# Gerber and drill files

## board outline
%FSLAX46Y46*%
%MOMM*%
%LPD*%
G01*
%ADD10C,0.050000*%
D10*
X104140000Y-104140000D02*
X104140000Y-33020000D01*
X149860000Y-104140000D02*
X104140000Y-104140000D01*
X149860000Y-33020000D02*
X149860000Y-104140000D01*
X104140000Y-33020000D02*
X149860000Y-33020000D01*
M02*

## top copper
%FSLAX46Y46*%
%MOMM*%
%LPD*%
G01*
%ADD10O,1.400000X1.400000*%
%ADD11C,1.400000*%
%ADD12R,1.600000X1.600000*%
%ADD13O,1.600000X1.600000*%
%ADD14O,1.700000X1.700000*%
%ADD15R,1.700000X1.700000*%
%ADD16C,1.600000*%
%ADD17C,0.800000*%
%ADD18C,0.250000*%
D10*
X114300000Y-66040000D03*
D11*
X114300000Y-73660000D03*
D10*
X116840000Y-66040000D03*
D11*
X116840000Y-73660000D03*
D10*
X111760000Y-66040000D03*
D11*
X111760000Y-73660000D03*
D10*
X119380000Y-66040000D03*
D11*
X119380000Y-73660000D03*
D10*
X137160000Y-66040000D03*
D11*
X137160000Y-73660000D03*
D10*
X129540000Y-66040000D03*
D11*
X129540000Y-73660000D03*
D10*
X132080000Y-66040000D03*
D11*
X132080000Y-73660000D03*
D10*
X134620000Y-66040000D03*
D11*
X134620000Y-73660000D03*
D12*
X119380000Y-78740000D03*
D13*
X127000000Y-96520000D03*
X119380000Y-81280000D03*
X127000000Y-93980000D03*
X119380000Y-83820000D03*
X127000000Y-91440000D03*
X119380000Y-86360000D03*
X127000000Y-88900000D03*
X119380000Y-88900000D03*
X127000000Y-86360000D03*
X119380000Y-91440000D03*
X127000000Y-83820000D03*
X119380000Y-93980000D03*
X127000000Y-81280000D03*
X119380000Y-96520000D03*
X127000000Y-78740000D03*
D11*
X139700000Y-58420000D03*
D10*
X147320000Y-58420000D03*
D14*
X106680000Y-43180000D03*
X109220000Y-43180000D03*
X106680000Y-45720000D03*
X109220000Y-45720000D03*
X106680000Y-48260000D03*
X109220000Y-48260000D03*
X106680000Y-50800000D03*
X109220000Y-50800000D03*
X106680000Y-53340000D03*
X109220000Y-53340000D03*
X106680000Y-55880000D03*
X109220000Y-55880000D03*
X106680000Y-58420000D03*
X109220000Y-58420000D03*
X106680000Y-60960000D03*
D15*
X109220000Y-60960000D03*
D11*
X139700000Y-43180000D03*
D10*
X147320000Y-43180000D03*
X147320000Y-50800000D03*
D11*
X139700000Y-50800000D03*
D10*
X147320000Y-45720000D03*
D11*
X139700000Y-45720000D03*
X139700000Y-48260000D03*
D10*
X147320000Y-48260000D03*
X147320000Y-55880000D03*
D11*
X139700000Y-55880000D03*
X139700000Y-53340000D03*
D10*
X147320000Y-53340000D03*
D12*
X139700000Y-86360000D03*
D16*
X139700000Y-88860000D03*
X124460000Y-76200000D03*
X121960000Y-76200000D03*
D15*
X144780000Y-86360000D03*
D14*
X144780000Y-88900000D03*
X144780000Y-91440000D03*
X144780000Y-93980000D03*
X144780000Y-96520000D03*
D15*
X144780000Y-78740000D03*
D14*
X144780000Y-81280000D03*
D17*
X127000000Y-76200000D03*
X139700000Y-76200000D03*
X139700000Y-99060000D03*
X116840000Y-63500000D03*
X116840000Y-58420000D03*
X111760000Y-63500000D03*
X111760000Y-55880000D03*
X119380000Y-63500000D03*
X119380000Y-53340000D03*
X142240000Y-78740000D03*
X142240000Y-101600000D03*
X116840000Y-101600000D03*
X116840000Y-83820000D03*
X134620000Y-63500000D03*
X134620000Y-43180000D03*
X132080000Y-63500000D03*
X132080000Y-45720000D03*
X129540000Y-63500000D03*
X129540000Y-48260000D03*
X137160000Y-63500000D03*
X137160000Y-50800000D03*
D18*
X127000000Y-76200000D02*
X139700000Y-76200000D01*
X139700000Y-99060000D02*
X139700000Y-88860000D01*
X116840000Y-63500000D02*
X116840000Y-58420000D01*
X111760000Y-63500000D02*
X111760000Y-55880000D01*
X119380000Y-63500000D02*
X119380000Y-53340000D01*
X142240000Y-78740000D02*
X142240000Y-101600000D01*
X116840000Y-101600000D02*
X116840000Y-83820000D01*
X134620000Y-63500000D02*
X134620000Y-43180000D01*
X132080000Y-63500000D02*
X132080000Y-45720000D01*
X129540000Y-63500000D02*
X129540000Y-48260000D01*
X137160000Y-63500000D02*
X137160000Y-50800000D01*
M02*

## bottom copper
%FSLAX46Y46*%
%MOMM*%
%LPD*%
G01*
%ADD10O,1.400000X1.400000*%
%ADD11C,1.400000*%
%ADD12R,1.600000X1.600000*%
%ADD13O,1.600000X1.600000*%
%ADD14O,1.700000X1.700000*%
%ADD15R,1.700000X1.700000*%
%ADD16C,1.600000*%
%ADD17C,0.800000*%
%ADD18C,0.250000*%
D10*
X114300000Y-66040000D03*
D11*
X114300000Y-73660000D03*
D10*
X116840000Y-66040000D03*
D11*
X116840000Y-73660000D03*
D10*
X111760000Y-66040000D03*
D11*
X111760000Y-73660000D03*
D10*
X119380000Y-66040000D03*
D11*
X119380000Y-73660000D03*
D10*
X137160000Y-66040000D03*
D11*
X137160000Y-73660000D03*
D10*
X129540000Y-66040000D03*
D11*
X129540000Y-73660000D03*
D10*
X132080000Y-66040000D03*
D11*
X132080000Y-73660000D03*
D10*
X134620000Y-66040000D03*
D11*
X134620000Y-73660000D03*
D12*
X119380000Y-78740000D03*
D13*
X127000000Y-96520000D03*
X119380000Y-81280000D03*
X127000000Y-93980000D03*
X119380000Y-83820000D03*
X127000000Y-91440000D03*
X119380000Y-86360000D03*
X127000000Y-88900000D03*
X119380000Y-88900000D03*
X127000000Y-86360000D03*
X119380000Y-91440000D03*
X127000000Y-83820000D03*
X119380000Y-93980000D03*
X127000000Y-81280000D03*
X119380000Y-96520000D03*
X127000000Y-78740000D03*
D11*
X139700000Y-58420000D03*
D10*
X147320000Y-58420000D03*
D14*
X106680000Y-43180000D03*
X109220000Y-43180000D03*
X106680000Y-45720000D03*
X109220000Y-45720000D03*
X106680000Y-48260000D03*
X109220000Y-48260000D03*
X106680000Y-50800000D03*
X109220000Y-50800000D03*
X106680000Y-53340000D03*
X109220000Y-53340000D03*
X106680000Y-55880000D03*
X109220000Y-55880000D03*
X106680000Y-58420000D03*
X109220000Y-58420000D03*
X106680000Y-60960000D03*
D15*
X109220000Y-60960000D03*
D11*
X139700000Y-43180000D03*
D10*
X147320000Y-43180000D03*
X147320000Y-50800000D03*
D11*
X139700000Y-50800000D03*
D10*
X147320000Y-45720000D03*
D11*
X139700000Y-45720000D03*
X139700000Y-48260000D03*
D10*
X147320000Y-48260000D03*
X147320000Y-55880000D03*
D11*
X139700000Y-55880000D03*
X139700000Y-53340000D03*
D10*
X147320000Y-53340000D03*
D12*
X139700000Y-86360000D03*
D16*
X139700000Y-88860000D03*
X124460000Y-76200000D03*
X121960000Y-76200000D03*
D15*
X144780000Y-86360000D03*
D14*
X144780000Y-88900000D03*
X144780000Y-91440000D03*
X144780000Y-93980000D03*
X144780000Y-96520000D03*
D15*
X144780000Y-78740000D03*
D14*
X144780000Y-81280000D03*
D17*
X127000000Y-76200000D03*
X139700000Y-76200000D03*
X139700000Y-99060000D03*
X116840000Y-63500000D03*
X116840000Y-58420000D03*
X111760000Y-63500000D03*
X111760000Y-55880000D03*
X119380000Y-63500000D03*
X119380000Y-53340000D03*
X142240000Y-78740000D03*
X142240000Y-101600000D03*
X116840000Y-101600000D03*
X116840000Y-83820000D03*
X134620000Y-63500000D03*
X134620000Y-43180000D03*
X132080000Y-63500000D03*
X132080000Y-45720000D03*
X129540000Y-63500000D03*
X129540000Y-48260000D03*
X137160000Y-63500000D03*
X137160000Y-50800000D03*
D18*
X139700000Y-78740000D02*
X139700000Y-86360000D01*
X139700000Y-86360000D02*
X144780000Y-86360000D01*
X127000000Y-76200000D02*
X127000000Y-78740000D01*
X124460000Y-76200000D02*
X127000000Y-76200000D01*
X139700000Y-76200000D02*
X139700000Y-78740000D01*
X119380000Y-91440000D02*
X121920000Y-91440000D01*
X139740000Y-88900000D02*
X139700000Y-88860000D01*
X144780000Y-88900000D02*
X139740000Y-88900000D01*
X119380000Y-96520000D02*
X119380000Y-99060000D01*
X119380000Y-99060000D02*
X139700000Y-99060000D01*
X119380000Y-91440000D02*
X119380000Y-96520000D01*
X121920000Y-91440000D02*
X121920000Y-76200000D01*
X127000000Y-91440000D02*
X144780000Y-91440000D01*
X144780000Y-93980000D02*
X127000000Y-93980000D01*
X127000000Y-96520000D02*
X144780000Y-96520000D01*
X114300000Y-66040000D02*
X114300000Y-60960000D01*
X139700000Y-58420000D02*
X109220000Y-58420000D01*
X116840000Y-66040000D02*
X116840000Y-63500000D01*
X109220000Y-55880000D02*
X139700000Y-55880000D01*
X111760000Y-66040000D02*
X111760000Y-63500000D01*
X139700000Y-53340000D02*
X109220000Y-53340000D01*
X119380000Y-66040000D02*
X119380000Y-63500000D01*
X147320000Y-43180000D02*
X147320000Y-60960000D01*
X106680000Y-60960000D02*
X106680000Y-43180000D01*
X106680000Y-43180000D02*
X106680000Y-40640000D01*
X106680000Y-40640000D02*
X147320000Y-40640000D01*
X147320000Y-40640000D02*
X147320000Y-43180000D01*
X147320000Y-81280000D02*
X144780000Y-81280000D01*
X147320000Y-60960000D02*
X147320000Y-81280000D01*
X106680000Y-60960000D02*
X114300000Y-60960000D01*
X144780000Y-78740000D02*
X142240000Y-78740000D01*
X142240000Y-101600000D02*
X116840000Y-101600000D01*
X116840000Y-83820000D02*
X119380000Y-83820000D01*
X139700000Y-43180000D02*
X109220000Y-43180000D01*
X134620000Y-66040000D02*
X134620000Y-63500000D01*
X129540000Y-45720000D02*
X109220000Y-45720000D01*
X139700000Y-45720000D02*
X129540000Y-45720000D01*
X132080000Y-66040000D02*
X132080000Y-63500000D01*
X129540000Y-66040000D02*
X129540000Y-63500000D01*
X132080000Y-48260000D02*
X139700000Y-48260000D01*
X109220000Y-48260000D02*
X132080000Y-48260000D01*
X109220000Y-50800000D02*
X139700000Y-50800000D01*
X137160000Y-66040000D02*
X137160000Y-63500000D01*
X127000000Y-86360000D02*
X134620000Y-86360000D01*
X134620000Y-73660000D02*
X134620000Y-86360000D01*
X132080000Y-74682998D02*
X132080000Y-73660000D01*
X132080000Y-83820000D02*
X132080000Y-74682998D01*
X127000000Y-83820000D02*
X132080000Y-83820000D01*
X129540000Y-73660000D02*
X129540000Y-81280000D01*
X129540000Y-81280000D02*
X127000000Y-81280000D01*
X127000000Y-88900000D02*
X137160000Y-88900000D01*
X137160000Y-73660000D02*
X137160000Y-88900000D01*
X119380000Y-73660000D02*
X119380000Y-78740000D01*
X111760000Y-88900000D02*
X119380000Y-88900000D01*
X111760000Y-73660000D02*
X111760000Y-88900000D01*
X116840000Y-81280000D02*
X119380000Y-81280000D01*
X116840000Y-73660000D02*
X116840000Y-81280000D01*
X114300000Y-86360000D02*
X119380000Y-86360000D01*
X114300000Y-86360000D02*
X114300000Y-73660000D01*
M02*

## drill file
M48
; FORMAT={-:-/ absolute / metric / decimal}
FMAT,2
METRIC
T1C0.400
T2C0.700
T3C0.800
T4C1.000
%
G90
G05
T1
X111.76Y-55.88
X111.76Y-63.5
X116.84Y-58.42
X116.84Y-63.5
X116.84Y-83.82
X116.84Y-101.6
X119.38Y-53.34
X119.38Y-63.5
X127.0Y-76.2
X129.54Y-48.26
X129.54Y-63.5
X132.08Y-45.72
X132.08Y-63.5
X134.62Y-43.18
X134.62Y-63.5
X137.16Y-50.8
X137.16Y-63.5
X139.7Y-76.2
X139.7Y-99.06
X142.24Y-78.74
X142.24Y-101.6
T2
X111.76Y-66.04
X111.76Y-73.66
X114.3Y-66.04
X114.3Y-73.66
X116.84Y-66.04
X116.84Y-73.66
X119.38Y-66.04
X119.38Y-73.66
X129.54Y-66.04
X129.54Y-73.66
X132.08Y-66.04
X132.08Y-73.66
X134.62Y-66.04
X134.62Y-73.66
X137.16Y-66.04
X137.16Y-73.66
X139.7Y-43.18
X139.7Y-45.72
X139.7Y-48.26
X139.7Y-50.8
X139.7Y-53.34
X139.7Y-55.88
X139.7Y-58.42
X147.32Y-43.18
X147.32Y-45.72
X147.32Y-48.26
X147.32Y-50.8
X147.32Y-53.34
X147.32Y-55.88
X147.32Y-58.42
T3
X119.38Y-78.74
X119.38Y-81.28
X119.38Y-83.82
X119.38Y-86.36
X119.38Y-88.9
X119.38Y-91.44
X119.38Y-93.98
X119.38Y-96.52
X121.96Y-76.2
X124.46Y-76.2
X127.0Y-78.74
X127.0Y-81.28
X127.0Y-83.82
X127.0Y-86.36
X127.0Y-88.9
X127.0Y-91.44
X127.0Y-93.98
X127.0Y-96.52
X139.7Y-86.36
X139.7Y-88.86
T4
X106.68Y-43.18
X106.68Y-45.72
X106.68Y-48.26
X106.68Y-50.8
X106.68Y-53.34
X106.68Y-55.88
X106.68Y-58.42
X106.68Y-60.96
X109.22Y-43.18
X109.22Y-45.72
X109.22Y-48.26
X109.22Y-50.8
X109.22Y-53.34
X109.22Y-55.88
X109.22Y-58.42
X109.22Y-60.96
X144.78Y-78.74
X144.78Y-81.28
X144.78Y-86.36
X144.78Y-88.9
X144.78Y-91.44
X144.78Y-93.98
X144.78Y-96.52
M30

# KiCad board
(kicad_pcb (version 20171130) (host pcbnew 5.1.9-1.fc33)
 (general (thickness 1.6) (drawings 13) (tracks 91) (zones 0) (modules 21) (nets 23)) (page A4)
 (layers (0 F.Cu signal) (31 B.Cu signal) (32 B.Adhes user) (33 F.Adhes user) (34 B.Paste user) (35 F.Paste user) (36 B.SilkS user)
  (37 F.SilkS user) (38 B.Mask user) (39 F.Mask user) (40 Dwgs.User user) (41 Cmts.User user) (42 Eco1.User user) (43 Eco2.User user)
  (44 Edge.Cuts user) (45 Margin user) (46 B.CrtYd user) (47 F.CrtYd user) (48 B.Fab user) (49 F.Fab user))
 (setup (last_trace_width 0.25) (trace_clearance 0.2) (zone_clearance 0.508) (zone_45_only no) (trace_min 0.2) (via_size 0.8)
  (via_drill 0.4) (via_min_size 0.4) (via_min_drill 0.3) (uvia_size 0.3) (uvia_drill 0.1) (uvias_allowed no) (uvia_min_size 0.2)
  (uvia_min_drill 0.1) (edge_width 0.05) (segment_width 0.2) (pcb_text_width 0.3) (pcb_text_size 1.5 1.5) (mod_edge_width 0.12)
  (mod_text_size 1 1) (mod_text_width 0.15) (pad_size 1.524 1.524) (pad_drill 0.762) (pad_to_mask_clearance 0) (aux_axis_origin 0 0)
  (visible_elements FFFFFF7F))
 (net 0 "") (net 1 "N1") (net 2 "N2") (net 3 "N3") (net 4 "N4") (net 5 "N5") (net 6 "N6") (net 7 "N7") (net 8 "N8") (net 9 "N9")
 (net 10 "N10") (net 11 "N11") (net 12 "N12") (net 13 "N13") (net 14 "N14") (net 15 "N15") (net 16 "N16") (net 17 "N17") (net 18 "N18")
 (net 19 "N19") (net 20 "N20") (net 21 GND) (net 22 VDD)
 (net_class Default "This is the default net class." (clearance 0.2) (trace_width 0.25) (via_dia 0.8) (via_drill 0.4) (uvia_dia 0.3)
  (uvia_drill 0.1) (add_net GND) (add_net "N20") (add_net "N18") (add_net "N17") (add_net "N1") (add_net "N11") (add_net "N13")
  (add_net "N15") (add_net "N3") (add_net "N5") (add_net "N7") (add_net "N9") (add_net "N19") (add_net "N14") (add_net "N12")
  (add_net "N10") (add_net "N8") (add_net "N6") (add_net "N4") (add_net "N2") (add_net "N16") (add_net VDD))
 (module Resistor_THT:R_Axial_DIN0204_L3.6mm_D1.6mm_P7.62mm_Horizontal (layer F.Cu) (at 114.3 73.66 90)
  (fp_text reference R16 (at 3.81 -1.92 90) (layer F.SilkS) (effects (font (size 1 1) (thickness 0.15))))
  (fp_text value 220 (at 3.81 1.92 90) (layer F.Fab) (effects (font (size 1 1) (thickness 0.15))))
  (pad 2 thru_hole oval (at 7.62 0 90) (size 1.4 1.4) (drill 0.7) (layers *.Cu *.Mask) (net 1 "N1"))
  (pad 1 thru_hole circle (at 0 0 90) (size 1.4 1.4) (drill 0.7) (layers *.Cu *.Mask) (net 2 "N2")))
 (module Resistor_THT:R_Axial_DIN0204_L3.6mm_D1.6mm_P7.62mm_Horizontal (layer F.Cu) (at 116.84 73.66 90)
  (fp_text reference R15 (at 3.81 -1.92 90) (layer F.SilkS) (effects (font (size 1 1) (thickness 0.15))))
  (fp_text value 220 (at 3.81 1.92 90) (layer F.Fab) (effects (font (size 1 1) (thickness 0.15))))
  (pad 2 thru_hole oval (at 7.62 0 90) (size 1.4 1.4) (drill 0.7) (layers *.Cu *.Mask) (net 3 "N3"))
  (pad 1 thru_hole circle (at 0 0 90) (size 1.4 1.4) (drill 0.7) (layers *.Cu *.Mask) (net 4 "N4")))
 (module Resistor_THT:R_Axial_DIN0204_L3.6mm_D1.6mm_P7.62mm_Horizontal (layer F.Cu) (at 111.76 73.66 90)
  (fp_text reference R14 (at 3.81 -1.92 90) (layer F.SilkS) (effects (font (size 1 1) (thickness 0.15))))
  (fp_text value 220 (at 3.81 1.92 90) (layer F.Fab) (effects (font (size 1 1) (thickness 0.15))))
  (pad 2 thru_hole oval (at 7.62 0 90) (size 1.4 1.4) (drill 0.7) (layers *.Cu *.Mask) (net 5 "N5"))
  (pad 1 thru_hole circle (at 0 0 90) (size 1.4 1.4) (drill 0.7) (layers *.Cu *.Mask) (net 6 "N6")))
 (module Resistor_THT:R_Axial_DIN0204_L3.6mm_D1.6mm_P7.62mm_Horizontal (layer F.Cu) (at 119.38 73.66 90)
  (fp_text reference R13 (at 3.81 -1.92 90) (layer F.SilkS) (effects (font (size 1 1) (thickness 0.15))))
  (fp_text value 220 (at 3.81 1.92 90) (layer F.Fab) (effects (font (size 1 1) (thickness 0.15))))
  (pad 2 thru_hole oval (at 7.62 0 90) (size 1.4 1.4) (drill 0.7) (layers *.Cu *.Mask) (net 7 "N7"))
  (pad 1 thru_hole circle (at 0 0 90) (size 1.4 1.4) (drill 0.7) (layers *.Cu *.Mask) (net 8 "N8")))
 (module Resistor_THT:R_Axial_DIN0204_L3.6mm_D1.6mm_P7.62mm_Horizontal (layer F.Cu) (at 137.16 73.66 90)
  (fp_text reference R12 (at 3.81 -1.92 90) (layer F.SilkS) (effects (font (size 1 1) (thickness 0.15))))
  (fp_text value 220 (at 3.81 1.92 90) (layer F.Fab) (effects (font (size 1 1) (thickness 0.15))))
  (pad 2 thru_hole oval (at 7.62 0 90) (size 1.4 1.4) (drill 0.7) (layers *.Cu *.Mask) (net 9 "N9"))
  (pad 1 thru_hole circle (at 0 0 90) (size 1.4 1.4) (drill 0.7) (layers *.Cu *.Mask) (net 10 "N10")))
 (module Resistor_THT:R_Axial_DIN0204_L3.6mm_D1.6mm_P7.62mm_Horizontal (layer F.Cu) (at 129.54 73.66 90)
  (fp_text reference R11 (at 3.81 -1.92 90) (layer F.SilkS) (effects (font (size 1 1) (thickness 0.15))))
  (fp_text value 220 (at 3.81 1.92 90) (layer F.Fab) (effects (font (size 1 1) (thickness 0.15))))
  (pad 2 thru_hole oval (at 7.62 0 90) (size 1.4 1.4) (drill 0.7) (layers *.Cu *.Mask) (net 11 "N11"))
  (pad 1 thru_hole circle (at 0 0 90) (size 1.4 1.4) (drill 0.7) (layers *.Cu *.Mask) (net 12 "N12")))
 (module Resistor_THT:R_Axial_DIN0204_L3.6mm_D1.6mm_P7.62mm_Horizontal (layer F.Cu) (at 132.08 73.66 90)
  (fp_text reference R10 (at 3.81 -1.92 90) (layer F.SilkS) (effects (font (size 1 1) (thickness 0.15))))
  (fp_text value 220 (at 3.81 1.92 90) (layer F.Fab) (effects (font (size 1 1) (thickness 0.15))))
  (pad 2 thru_hole oval (at 7.62 0 90) (size 1.4 1.4) (drill 0.7) (layers *.Cu *.Mask) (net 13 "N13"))
  (pad 1 thru_hole circle (at 0 0 90) (size 1.4 1.4) (drill 0.7) (layers *.Cu *.Mask) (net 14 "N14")))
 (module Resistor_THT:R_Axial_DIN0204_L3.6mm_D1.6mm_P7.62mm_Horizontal (layer F.Cu) (at 134.62 73.66 90)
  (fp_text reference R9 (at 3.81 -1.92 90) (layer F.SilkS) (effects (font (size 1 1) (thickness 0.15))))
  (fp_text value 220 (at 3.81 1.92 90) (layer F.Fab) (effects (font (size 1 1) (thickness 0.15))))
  (pad 2 thru_hole oval (at 7.62 0 90) (size 1.4 1.4) (drill 0.7) (layers *.Cu *.Mask) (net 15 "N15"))
  (pad 1 thru_hole circle (at 0 0 90) (size 1.4 1.4) (drill 0.7) (layers *.Cu *.Mask) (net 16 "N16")))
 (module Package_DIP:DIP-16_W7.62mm (layer F.Cu) (at 119.38 78.74)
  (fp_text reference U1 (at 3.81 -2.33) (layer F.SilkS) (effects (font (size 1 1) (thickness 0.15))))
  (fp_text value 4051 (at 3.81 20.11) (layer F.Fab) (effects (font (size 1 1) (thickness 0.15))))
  (pad 1 thru_hole rect (at 0 0) (size 1.6 1.6) (drill 0.8) (layers *.Cu *.Mask) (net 8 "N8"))
  (pad 9 thru_hole oval (at 7.62 17.78) (size 1.6 1.6) (drill 0.8) (layers *.Cu *.Mask) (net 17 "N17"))
  (pad 2 thru_hole oval (at 0 2.54) (size 1.6 1.6) (drill 0.8) (layers *.Cu *.Mask) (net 4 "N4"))
  (pad 10 thru_hole oval (at 7.62 15.24) (size 1.6 1.6) (drill 0.8) (layers *.Cu *.Mask) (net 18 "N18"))
  (pad 3 thru_hole oval (at 0 5.08) (size 1.6 1.6) (drill 0.8) (layers *.Cu *.Mask) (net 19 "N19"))
  (pad 11 thru_hole oval (at 7.62 12.7) (size 1.6 1.6) (drill 0.8) (layers *.Cu *.Mask) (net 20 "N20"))
  (pad 4 thru_hole oval (at 0 7.62) (size 1.6 1.6) (drill 0.8) (layers *.Cu *.Mask) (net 2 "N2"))
  (pad 12 thru_hole oval (at 7.62 10.16) (size 1.6 1.6) (drill 0.8) (layers *.Cu *.Mask) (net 10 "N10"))
  (pad 5 thru_hole oval (at 0 10.16) (size 1.6 1.6) (drill 0.8) (layers *.Cu *.Mask) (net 6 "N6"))
  (pad 13 thru_hole oval (at 7.62 7.62) (size 1.6 1.6) (drill 0.8) (layers *.Cu *.Mask) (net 16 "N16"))
  (pad 6 thru_hole oval (at 0 12.7) (size 1.6 1.6) (drill 0.8) (layers *.Cu *.Mask) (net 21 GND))
  (pad 14 thru_hole oval (at 7.62 5.08) (size 1.6 1.6) (drill 0.8) (layers *.Cu *.Mask) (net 14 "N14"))
  (pad 7 thru_hole oval (at 0 15.24) (size 1.6 1.6) (drill 0.8) (layers *.Cu *.Mask) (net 21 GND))
  (pad 15 thru_hole oval (at 7.62 2.54) (size 1.6 1.6) (drill 0.8) (layers *.Cu *.Mask) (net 12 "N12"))
  (pad 8 thru_hole oval (at 0 17.78) (size 1.6 1.6) (drill 0.8) (layers *.Cu *.Mask) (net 21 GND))
  (pad 16 thru_hole oval (at 7.62 0) (size 1.6 1.6) (drill 0.8) (layers *.Cu *.Mask) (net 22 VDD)))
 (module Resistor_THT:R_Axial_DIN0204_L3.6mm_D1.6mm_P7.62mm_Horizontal (layer F.Cu) (at 139.7 58.42)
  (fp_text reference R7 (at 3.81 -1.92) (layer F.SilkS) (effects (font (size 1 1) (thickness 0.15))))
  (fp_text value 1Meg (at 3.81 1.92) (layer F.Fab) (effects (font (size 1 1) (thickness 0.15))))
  (pad 1 thru_hole circle (at 0 0) (size 1.4 1.4) (drill 0.7) (layers *.Cu *.Mask) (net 3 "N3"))
  (pad 2 thru_hole oval (at 7.62 0) (size 1.4 1.4) (drill 0.7) (layers *.Cu *.Mask) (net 1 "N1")))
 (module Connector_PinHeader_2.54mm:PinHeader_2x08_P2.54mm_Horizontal (layer F.Cu) (at 109.22 60.96 180)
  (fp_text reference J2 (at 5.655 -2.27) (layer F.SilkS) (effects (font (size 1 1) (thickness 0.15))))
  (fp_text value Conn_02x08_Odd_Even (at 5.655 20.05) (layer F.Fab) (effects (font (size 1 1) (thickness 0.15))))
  (pad 16 thru_hole oval (at 2.54 17.78 180) (size 1.7 1.7) (drill 1) (layers *.Cu *.Mask) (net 1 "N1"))
  (pad 15 thru_hole oval (at 0 17.78 180) (size 1.7 1.7) (drill 1) (layers *.Cu *.Mask) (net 15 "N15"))
  (pad 14 thru_hole oval (at 2.54 15.24 180) (size 1.7 1.7) (drill 1) (layers *.Cu *.Mask) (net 1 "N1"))
  (pad 13 thru_hole oval (at 0 15.24 180) (size 1.7 1.7) (drill 1) (layers *.Cu *.Mask) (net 13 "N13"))
  (pad 12 thru_hole oval (at 2.54 12.7 180) (size 1.7 1.7) (drill 1) (layers *.Cu *.Mask) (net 1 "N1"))
  (pad 11 thru_hole oval (at 0 12.7 180) (size 1.7 1.7) (drill 1) (layers *.Cu *.Mask) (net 11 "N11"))
  (pad 10 thru_hole oval (at 2.54 10.16 180) (size 1.7 1.7) (drill 1) (layers *.Cu *.Mask) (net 1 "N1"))
  (pad 9 thru_hole oval (at 0 10.16 180) (size 1.7 1.7) (drill 1) (layers *.Cu *.Mask) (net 9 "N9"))
  (pad 8 thru_hole oval (at 2.54 7.62 180) (size 1.7 1.7) (drill 1) (layers *.Cu *.Mask) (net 1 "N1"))
  (pad 7 thru_hole oval (at 0 7.62 180) (size 1.7 1.7) (drill 1) (layers *.Cu *.Mask) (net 7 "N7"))
  (pad 6 thru_hole oval (at 2.54 5.08 180) (size 1.7 1.7) (drill 1) (layers *.Cu *.Mask) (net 1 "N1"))
  (pad 5 thru_hole oval (at 0 5.08 180) (size 1.7 1.7) (drill 1) (layers *.Cu *.Mask) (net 5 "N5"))
  (pad 4 thru_hole oval (at 2.54 2.54 180) (size 1.7 1.7) (drill 1) (layers *.Cu *.Mask) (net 1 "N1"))
  (pad 3 thru_hole oval (at 0 2.54 180) (size 1.7 1.7) (drill 1) (layers *.Cu *.Mask) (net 3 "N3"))
  (pad 2 thru_hole oval (at 2.54 0 180) (size 1.7 1.7) (drill 1) (layers *.Cu *.Mask) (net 1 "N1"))
  (pad 1 thru_hole rect (at 0 0 180) (size 1.7 1.7) (drill 1) (layers *.Cu *.Mask) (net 1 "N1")))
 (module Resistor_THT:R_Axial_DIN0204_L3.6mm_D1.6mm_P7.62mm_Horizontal (layer F.Cu) (at 139.7 43.18)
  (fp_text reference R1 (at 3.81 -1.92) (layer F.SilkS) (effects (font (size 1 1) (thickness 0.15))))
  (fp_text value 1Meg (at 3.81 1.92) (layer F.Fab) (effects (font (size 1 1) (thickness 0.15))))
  (pad 1 thru_hole circle (at 0 0) (size 1.4 1.4) (drill 0.7) (layers *.Cu *.Mask) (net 15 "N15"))
  (pad 2 thru_hole oval (at 7.62 0) (size 1.4 1.4) (drill 0.7) (layers *.Cu *.Mask) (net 1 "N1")))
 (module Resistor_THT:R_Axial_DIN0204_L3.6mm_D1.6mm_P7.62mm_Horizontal (layer F.Cu) (at 139.7 50.8)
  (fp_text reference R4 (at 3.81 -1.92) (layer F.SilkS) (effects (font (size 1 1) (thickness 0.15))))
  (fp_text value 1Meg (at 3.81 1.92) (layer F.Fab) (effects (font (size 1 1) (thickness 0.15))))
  (pad 2 thru_hole oval (at 7.62 0) (size 1.4 1.4) (drill 0.7) (layers *.Cu *.Mask) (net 1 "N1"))
  (pad 1 thru_hole circle (at 0 0) (size 1.4 1.4) (drill 0.7) (layers *.Cu *.Mask) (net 9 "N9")))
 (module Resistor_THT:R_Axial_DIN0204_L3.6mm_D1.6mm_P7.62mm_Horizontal (layer F.Cu) (at 139.7 45.72)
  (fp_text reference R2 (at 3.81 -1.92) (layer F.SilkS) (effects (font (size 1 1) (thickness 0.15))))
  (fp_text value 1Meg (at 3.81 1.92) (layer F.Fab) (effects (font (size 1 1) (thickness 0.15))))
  (pad 2 thru_hole oval (at 7.62 0) (size 1.4 1.4) (drill 0.7) (layers *.Cu *.Mask) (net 1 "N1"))
  (pad 1 thru_hole circle (at 0 0) (size 1.4 1.4) (drill 0.7) (layers *.Cu *.Mask) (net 13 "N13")))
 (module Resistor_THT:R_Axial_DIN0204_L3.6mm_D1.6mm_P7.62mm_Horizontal (layer F.Cu) (at 139.7 48.26)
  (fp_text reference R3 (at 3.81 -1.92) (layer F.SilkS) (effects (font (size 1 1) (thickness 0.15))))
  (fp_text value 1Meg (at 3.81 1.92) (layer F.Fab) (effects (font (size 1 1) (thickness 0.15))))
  (pad 1 thru_hole circle (at 0 0) (size 1.4 1.4) (drill 0.7) (layers *.Cu *.Mask) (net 11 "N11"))
  (pad 2 thru_hole oval (at 7.62 0) (size 1.4 1.4) (drill 0.7) (layers *.Cu *.Mask) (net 1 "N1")))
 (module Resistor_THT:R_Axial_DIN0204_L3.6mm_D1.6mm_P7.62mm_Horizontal (layer F.Cu) (at 139.7 55.88)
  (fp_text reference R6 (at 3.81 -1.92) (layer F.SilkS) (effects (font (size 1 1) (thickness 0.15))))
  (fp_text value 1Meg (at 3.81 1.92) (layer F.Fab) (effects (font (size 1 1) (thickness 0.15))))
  (pad 2 thru_hole oval (at 7.62 0) (size 1.4 1.4) (drill 0.7) (layers *.Cu *.Mask) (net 1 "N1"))
  (pad 1 thru_hole circle (at 0 0) (size 1.4 1.4) (drill 0.7) (layers *.Cu *.Mask) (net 5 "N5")))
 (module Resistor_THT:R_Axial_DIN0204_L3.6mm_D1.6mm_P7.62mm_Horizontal (layer F.Cu) (at 139.7 53.34)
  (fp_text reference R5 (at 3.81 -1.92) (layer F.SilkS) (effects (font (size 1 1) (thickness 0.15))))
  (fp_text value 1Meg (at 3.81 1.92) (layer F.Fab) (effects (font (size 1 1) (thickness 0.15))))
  (pad 1 thru_hole circle (at 0 0) (size 1.4 1.4) (drill 0.7) (layers *.Cu *.Mask) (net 7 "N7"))
  (pad 2 thru_hole oval (at 7.62 0) (size 1.4 1.4) (drill 0.7) (layers *.Cu *.Mask) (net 1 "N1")))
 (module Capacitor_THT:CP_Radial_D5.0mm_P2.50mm (layer F.Cu) (at 139.7 86.36 270)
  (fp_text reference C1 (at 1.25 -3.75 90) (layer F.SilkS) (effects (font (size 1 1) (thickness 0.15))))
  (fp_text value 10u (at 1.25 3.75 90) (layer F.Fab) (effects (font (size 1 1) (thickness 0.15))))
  (pad 1 thru_hole rect (at 0 0 270) (size 1.6 1.6) (drill 0.8) (layers *.Cu *.Mask) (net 22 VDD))
  (pad 2 thru_hole circle (at 2.5 0 270) (size 1.6 1.6) (drill 0.8) (layers *.Cu *.Mask) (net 21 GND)))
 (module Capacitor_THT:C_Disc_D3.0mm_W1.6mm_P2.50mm (layer F.Cu) (at 124.46 76.2 180)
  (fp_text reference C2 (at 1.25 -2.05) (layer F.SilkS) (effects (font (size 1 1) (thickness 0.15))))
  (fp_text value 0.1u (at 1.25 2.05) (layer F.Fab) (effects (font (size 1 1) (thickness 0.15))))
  (pad 1 thru_hole circle (at 0 0 180) (size 1.6 1.6) (drill 0.8) (layers *.Cu *.Mask) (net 22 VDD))
  (pad 2 thru_hole circle (at 2.5 0 180) (size 1.6 1.6) (drill 0.8) (layers *.Cu *.Mask) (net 21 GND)))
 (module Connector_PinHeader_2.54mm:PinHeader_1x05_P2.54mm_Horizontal (layer F.Cu) (at 144.78 86.36)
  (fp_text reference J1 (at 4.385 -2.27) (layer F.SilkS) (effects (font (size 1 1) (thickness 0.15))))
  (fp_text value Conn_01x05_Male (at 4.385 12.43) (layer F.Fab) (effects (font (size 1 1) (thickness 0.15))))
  (pad 1 thru_hole rect (at 0 0) (size 1.7 1.7) (drill 1) (layers *.Cu *.Mask) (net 22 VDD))
  (pad 2 thru_hole oval (at 0 2.54) (size 1.7 1.7) (drill 1) (layers *.Cu *.Mask) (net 21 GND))
  (pad 3 thru_hole oval (at 0 5.08) (size 1.7 1.7) (drill 1) (layers *.Cu *.Mask) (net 20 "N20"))
  (pad 4 thru_hole oval (at 0 7.62) (size 1.7 1.7) (drill 1) (layers *.Cu *.Mask) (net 18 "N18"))
  (pad 5 thru_hole oval (at 0 10.16) (size 1.7 1.7) (drill 1) (layers *.Cu *.Mask) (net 17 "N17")))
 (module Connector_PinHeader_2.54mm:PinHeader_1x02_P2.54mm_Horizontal (layer F.Cu) (at 144.78 78.74)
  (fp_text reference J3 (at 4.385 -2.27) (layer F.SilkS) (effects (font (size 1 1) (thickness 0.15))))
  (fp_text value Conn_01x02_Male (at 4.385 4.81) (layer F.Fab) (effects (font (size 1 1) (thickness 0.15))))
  (pad 1 thru_hole rect (at 0 0) (size 1.7 1.7) (drill 1) (layers *.Cu *.Mask) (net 19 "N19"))
  (pad 2 thru_hole oval (at 0 2.54) (size 1.7 1.7) (drill 1) (layers *.Cu *.Mask) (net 1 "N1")))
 (gr_line (start 104.14 104.14) (end 104.14 33.02) (layer Edge.Cuts) (width 0.05))
 (gr_line (start 149.86 104.14) (end 104.14 104.14) (layer Edge.Cuts) (width 0.05))
 (gr_line (start 149.86 33.02) (end 149.86 104.14) (layer Edge.Cuts) (width 0.05))
 (gr_line (start 104.14 33.02) (end 149.86 33.02) (layer Edge.Cuts) (width 0.05))
 (segment (start 139.7 78.74) (end 139.7 86.36) (width 0.25) (layer B.Cu) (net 22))
 (segment (start 139.7 86.36) (end 144.78 86.36) (width 0.25) (layer B.Cu) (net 22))
 (segment (start 127 76.2) (end 127 78.74) (width 0.25) (layer B.Cu) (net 22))
 (via (at 127 76.2) (size 0.8) (drill 0.4) (layers F.Cu B.Cu) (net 22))
 (segment (start 124.46 76.2) (end 127 76.2) (width 0.25) (layer B.Cu) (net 22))
 (via (at 139.7 76.2) (size 0.8) (drill 0.4) (layers F.Cu B.Cu) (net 22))
 (segment (start 127 76.2) (end 139.7 76.2) (width 0.25) (layer F.Cu) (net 22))
 (segment (start 139.7 76.2) (end 139.7 78.74) (width 0.25) (layer B.Cu) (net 22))
 (segment (start 119.38 91.44) (end 121.92 91.44) (width 0.25) (layer B.Cu) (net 21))
 (segment (start 139.74 88.9) (end 139.7 88.86) (width 0.25) (layer B.Cu) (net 21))
 (segment (start 144.78 88.9) (end 139.74 88.9) (width 0.25) (layer B.Cu) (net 21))
 (segment (start 119.38 96.52) (end 119.38 99.06) (width 0.25) (layer B.Cu) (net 21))
 (via (at 139.7 99.06) (size 0.8) (drill 0.4) (layers F.Cu B.Cu) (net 21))
 (segment (start 119.38 99.06) (end 139.7 99.06) (width 0.25) (layer B.Cu) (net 21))
 (segment (start 139.7 99.06) (end 139.7 88.86) (width 0.25) (layer F.Cu) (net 21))
 (segment (start 119.38 91.44) (end 119.38 96.52) (width 0.25) (layer B.Cu) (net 21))
 (segment (start 121.92 91.44) (end 121.92 76.2) (width 0.25) (layer B.Cu) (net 21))
 (segment (start 127 91.44) (end 144.78 91.44) (width 0.25) (layer B.Cu) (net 20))
 (segment (start 144.78 93.98) (end 127 93.98) (width 0.25) (layer B.Cu) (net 18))
 (segment (start 127 96.52) (end 144.78 96.52) (width 0.25) (layer B.Cu) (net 17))
 (segment (start 114.3 66.04) (end 114.3 60.96) (width 0.25) (layer B.Cu) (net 1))
 (segment (start 139.7 58.42) (end 109.22 58.42) (width 0.25) (layer B.Cu) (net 3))
 (via (at 116.84 63.5) (size 0.8) (drill 0.4) (layers F.Cu B.Cu) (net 3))
 (segment (start 116.84 66.04) (end 116.84 63.5) (width 0.25) (layer B.Cu) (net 3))
 (via (at 116.84 58.42) (size 0.8) (drill 0.4) (layers F.Cu B.Cu) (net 3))
 (segment (start 116.84 63.5) (end 116.84 58.42) (width 0.25) (layer F.Cu) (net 3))
 (segment (start 109.22 55.88) (end 139.7 55.88) (width 0.25) (layer B.Cu) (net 5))
 (via (at 111.76 63.5) (size 0.8) (drill 0.4) (layers F.Cu B.Cu) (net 5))
 (segment (start 111.76 66.04) (end 111.76 63.5) (width 0.25) (layer B.Cu) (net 5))
 (segment (start 111.76 63.5) (end 111.76 55.88) (width 0.25) (layer F.Cu) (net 5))
 (via (at 111.76 55.88) (size 0.8) (drill 0.4) (layers F.Cu B.Cu) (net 5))
 (segment (start 139.7 53.34) (end 109.22 53.34) (width 0.25) (layer B.Cu) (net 7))
 (via (at 119.38 63.5) (size 0.8) (drill 0.4) (layers F.Cu B.Cu) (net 7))
 (segment (start 119.38 66.04) (end 119.38 63.5) (width 0.25) (layer B.Cu) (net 7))
 (via (at 119.38 53.34) (size 0.8) (drill 0.4) (layers F.Cu B.Cu) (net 7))
 (segment (start 119.38 63.5) (end 119.38 53.34) (width 0.25) (layer F.Cu) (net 7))
 (segment (start 147.32 43.18) (end 147.32 60.96) (width 0.25) (layer B.Cu) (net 1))
 (segment (start 106.68 60.96) (end 106.68 43.18) (width 0.25) (layer B.Cu) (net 1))
 (segment (start 106.68 43.18) (end 106.68 40.64) (width 0.25) (layer B.Cu) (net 1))
 (segment (start 106.68 40.64) (end 147.32 40.64) (width 0.25) (layer B.Cu) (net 1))
 (segment (start 147.32 40.64) (end 147.32 43.18) (width 0.25) (layer B.Cu) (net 1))
 (segment (start 147.32 81.28) (end 144.78 81.28) (width 0.25) (layer B.Cu) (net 1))
 (segment (start 147.32 60.96) (end 147.32 81.28) (width 0.25) (layer B.Cu) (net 1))
 (segment (start 106.68 60.96) (end 114.3 60.96) (width 0.25) (layer B.Cu) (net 1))
 (via (at 142.24 78.74) (size 0.8) (drill 0.4) (layers F.Cu B.Cu) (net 19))
 (segment (start 144.78 78.74) (end 142.24 78.74) (width 0.25) (layer B.Cu) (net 19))
 (via (at 142.24 101.6) (size 0.8) (drill 0.4) (layers F.Cu B.Cu) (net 19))
 (segment (start 142.24 78.74) (end 142.24 101.6) (width 0.25) (layer F.Cu) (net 19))
 (via (at 116.84 101.6) (size 0.8) (drill 0.4) (layers F.Cu B.Cu) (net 19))
 (segment (start 142.24 101.6) (end 116.84 101.6) (width 0.25) (layer B.Cu) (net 19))
 (via (at 116.84 83.82) (size 0.8) (drill 0.4) (layers F.Cu B.Cu) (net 19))
 (segment (start 116.84 101.6) (end 116.84 83.82) (width 0.25) (layer F.Cu) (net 19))
 (segment (start 116.84 83.82) (end 119.38 83.82) (width 0.25) (layer B.Cu) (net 19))
 (segment (start 139.7 43.18) (end 109.22 43.18) (width 0.25) (layer B.Cu) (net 15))
 (via (at 134.62 63.5) (size 0.8) (drill 0.4) (layers F.Cu B.Cu) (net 15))
 (segment (start 134.62 66.04) (end 134.62 63.5) (width 0.25) (layer B.Cu) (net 15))
 (via (at 134.62 43.18) (size 0.8) (drill 0.4) (layers F.Cu B.Cu) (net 15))
 (segment (start 134.62 63.5) (end 134.62 43.18) (width 0.25) (layer F.Cu) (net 15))
 (segment (start 129.54 45.72) (end 109.22 45.72) (width 0.25) (layer B.Cu) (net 13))
 (segment (start 139.7 45.72) (end 129.54 45.72) (width 0.25) (layer B.Cu) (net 13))
 (via (at 132.08 63.5) (size 0.8) (drill 0.4) (layers F.Cu B.Cu) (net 13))
 (segment (start 132.08 66.04) (end 132.08 63.5) (width 0.25) (layer B.Cu) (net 13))
 (via (at 132.08 45.72) (size 0.8) (drill 0.4) (layers F.Cu B.Cu) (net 13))
 (segment (start 132.08 63.5) (end 132.08 45.72) (width 0.25) (layer F.Cu) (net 13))
 (via (at 129.54 63.5) (size 0.8) (drill 0.4) (layers F.Cu B.Cu) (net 11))
 (segment (start 129.54 66.04) (end 129.54 63.5) (width 0.25) (layer B.Cu) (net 11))
 (segment (start 132.08 48.26) (end 139.7 48.26) (width 0.25) (layer B.Cu) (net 11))
 (segment (start 109.22 48.26) (end 132.08 48.26) (width 0.25) (layer B.Cu) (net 11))
 (via (at 129.54 48.26) (size 0.8) (drill 0.4) (layers F.Cu B.Cu) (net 11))
 (segment (start 129.54 63.5) (end 129.54 48.26) (width 0.25) (layer F.Cu) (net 11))
 (segment (start 109.22 50.8) (end 139.7 50.8) (width 0.25) (layer B.Cu) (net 9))
 (via (at 137.16 63.5) (size 0.8) (drill 0.4) (layers F.Cu B.Cu) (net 9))
 (segment (start 137.16 66.04) (end 137.16 63.5) (width 0.25) (layer B.Cu) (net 9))
 (via (at 137.16 50.8) (size 0.8) (drill 0.4) (layers F.Cu B.Cu) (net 9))
 (segment (start 137.16 63.5) (end 137.16 50.8) (width 0.25) (layer F.Cu) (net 9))
 (segment (start 127 86.36) (end 134.62 86.36) (width 0.25) (layer B.Cu) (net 16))
 (segment (start 134.62 73.66) (end 134.62 86.36) (width 0.25) (layer B.Cu) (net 16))
 (segment (start 132.08 74.682998) (end 132.08 73.66) (width 0.25) (layer B.Cu) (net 14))
 (segment (start 132.08 83.82) (end 132.08 74.682998) (width 0.25) (layer B.Cu) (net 14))
 (segment (start 127 83.82) (end 132.08 83.82) (width 0.25) (layer B.Cu) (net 14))
 (segment (start 129.54 73.66) (end 129.54 81.28) (width 0.25) (layer B.Cu) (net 12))
 (segment (start 129.54 81.28) (end 127 81.28) (width 0.25) (layer B.Cu) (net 12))
 (segment (start 127 88.9) (end 137.16 88.9) (width 0.25) (layer B.Cu) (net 10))
 (segment (start 137.16 73.66) (end 137.16 88.9) (width 0.25) (layer B.Cu) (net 10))
 (segment (start 119.38 73.66) (end 119.38 78.74) (width 0.25) (layer B.Cu) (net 8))
 (segment (start 111.76 88.9) (end 119.38 88.9) (width 0.25) (layer B.Cu) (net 6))
 (segment (start 111.76 73.66) (end 111.76 88.9) (width 0.25) (layer B.Cu) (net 6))
 (segment (start 116.84 81.28) (end 119.38 81.28) (width 0.25) (layer B.Cu) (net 4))
 (segment (start 116.84 73.66) (end 116.84 81.28) (width 0.25) (layer B.Cu) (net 4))
 (segment (start 114.3 86.36) (end 119.38 86.36) (width 0.25) (layer B.Cu) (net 2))
 (segment (start 114.3 86.36) (end 114.3 73.66) (width 0.25) (layer B.Cu) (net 2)))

